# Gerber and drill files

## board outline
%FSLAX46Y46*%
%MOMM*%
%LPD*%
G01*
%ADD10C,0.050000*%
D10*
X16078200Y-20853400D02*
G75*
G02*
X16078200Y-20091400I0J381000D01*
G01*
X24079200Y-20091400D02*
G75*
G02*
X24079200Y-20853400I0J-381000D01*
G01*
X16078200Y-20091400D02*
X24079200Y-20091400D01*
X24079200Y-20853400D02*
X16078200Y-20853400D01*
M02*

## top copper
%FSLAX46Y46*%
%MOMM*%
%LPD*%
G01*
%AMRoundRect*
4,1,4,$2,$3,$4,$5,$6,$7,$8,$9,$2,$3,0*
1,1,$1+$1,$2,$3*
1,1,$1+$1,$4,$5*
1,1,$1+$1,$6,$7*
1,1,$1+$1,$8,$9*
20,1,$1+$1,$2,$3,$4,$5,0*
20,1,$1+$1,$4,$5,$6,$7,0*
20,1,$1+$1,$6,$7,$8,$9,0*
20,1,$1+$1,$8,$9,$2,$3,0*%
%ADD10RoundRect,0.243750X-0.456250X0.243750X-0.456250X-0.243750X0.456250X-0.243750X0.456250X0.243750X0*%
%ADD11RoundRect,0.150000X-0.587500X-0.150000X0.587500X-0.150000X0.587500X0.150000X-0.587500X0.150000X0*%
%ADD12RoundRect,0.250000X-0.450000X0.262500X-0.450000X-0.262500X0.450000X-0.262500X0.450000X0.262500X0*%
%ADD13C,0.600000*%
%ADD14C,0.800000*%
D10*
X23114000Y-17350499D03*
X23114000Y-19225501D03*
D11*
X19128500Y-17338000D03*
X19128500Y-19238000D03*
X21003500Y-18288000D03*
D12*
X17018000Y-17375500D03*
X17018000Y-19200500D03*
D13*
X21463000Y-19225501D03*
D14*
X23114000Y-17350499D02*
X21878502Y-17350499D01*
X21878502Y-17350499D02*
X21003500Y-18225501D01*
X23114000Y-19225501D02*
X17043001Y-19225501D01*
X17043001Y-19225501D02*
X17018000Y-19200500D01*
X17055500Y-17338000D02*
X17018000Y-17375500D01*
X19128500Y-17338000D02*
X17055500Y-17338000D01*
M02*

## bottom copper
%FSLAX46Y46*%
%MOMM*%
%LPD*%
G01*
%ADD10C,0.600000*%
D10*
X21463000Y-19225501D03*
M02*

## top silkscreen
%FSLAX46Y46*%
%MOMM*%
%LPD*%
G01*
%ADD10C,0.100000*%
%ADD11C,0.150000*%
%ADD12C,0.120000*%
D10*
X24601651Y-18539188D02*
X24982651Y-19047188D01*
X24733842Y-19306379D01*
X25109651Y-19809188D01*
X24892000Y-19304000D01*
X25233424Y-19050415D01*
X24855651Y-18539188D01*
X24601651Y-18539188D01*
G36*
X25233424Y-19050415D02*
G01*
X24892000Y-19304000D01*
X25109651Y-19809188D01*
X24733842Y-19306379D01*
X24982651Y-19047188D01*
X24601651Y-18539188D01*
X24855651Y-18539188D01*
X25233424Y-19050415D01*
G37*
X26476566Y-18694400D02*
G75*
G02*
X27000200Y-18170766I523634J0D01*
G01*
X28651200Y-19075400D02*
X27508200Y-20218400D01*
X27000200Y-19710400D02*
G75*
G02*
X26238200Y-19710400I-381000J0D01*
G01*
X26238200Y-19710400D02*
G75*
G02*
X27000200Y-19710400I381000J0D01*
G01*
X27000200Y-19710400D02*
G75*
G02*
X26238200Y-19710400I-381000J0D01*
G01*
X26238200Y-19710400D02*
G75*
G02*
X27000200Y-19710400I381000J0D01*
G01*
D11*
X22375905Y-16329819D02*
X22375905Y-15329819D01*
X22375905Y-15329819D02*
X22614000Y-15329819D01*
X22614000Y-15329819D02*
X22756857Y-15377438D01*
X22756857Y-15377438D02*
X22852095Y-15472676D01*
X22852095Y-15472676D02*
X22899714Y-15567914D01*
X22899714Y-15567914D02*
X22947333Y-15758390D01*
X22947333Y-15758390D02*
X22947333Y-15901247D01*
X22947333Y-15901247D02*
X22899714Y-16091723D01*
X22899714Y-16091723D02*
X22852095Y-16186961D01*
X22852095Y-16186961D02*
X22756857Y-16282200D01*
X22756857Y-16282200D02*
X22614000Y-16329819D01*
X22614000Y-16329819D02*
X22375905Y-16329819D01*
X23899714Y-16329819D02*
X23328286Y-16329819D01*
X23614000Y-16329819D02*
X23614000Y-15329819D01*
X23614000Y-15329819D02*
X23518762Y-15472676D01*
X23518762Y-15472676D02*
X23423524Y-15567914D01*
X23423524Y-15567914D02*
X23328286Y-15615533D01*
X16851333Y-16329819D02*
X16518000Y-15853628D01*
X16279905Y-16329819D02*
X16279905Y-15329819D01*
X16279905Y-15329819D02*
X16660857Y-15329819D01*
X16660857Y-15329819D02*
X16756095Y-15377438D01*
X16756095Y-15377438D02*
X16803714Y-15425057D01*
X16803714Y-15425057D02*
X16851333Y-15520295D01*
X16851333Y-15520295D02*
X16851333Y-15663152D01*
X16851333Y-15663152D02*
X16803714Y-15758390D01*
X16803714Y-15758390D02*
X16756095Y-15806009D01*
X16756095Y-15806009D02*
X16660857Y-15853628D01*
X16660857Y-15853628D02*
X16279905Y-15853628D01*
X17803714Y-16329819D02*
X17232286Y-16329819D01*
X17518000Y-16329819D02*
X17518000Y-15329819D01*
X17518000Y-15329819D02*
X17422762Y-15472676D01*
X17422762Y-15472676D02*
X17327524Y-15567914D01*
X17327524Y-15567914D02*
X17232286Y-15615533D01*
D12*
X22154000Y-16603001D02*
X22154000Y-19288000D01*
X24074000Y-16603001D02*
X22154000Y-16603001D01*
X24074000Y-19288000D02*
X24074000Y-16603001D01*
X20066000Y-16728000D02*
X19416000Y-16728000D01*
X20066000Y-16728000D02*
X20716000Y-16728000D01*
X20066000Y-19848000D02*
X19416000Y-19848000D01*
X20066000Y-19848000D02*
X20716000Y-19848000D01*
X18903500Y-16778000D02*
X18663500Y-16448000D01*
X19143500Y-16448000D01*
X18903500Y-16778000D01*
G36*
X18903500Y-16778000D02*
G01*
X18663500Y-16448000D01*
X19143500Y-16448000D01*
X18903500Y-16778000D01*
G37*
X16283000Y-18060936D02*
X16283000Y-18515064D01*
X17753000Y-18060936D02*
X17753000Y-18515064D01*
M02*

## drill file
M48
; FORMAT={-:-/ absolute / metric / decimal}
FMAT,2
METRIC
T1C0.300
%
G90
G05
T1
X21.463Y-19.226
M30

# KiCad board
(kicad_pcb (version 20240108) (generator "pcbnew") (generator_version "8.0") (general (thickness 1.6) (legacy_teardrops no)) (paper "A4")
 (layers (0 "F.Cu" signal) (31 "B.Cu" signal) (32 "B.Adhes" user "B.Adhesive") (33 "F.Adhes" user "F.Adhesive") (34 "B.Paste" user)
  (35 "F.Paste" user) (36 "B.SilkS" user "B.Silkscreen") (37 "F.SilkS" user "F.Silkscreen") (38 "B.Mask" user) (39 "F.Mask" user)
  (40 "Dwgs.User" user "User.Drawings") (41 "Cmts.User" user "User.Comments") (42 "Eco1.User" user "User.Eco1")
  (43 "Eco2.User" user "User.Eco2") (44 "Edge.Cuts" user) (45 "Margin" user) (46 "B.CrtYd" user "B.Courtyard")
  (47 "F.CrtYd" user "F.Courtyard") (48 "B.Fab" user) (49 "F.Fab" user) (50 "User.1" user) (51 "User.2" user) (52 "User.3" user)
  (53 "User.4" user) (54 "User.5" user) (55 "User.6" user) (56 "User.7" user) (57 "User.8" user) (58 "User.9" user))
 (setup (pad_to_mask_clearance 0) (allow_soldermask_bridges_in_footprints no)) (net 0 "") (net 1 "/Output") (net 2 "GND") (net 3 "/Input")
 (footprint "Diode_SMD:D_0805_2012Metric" (layer "F.Cu") (at 23.114 18.288 -90)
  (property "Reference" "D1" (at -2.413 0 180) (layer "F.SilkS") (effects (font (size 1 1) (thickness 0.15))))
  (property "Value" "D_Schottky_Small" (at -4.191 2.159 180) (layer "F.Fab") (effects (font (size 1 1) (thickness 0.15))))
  (fp_line (start -1.684999 0.96) (end 1 0.96) (stroke (width 0.12) (type solid)) (layer "F.SilkS"))
  (fp_line (start -1.684999 -0.96) (end -1.684999 0.96) (stroke (width 0.12) (type solid)) (layer "F.SilkS"))
  (fp_line (start 1 -0.96) (end -1.684999 -0.96) (stroke (width 0.12) (type solid)) (layer "F.SilkS"))
  (pad "1" smd roundrect (at -0.937501 0 270) (size 0.975 1.4) (layers "F.Cu" "F.Paste" "F.Mask") (roundrect_rratio 0.25) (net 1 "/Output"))
  (pad "2" smd roundrect (at 0.937501 0 270) (size 0.975 1.4) (layers "F.Cu" "F.Paste" "F.Mask") (roundrect_rratio 0.25) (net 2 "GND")))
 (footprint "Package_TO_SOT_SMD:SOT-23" (layer "F.Cu") (at 20.066 18.288)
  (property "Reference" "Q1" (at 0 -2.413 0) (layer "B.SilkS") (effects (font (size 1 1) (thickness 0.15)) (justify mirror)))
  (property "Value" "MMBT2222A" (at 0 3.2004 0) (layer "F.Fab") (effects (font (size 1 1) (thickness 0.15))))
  (fp_line (start 0 -1.56) (end -0.65 -1.56) (stroke (width 0.12) (type solid)) (layer "F.SilkS"))
  (fp_line (start 0 -1.56) (end 0.65 -1.56) (stroke (width 0.12) (type solid)) (layer "F.SilkS"))
  (fp_line (start 0 1.56) (end -0.65 1.56) (stroke (width 0.12) (type solid)) (layer "F.SilkS"))
  (fp_line (start 0 1.56) (end 0.65 1.56) (stroke (width 0.12) (type solid)) (layer "F.SilkS"))
  (fp_poly
   (pts (xy -1.1625 -1.51) (xy -1.4025 -1.84) (xy -0.9225 -1.84) (xy -1.1625 -1.51)) (stroke (width 0.12) (type solid)) (fill solid)
   (layer "F.SilkS"))
  (pad "1" smd roundrect (at -0.9375 -0.95) (size 1.475 0.6) (layers "F.Cu" "F.Paste" "F.Mask") (roundrect_rratio 0.25) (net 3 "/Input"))
  (pad "2" smd roundrect (at -0.9375 0.95) (size 1.475 0.6) (layers "F.Cu" "F.Paste" "F.Mask") (roundrect_rratio 0.25) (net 2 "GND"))
  (pad "3" smd roundrect (at 0.9375 0) (size 1.475 0.6) (layers "F.Cu" "F.Paste" "F.Mask") (roundrect_rratio 0.25) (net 1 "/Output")))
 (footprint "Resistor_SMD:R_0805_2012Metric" (layer "F.Cu") (at 17.018 18.288 -90)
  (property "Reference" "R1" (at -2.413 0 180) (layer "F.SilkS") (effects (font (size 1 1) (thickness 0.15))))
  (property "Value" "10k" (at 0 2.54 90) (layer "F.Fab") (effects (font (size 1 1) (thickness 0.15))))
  (fp_line (start -0.227064 0.735) (end 0.227064 0.735) (stroke (width 0.12) (type solid)) (layer "F.SilkS"))
  (fp_line (start -0.227064 -0.735) (end 0.227064 -0.735) (stroke (width 0.12) (type solid)) (layer "F.SilkS"))
  (pad "1" smd roundrect (at -0.9125 0 270) (size 1.025 1.4) (layers "F.Cu" "F.Paste" "F.Mask") (roundrect_rratio 0.243902) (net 3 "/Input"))
  (pad "2" smd roundrect (at 0.9125 0 270) (size 1.025 1.4) (layers "F.Cu" "F.Paste" "F.Mask") (roundrect_rratio 0.243902) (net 2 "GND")))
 (gr_poly
  (pts (xy 24.601651 18.539188) (xy 24.982651 19.047188) (xy 24.733842 19.306379) (xy 25.109651 19.809188) (xy 24.892 19.304)
   (xy 25.233424 19.050415) (xy 24.855651 18.539188))
  (stroke (width 0.1) (type solid)) (fill solid) (layer "F.SilkS"))
 (gr_arc (start 26.476566 18.6944) (mid 26.629935 18.324135) (end 27.0002 18.170766) (stroke (width 0.1) (type default)) (layer "F.SilkS"))
 (gr_line (start 28.6512 19.0754) (end 27.5082 20.2184) (stroke (width 0.1) (type default)) (layer "F.SilkS"))
 (gr_circle (center 26.6192 19.7104) (end 26.6192 19.3294) (stroke (width 0.1) (type default)) (fill none) (layer "F.SilkS"))
 (gr_circle (center 26.6192 19.7104) (end 26.6192 19.3294) (stroke (width 0.1) (type default)) (fill none) (layer "F.SilkS"))
 (gr_arc (start 16.0782 20.8534) (mid 15.6972 20.4724) (end 16.0782 20.0914) (stroke (width 0.05) (type default)) (layer "Edge.Cuts"))
 (gr_arc (start 24.0792 20.0914) (mid 24.4602 20.4724) (end 24.0792 20.8534) (stroke (width 0.05) (type default)) (layer "Edge.Cuts"))
 (gr_line (start 16.0782 20.0914) (end 24.0792 20.0914) (stroke (width 0.05) (type default)) (layer "Edge.Cuts"))
 (gr_line (start 24.0792 20.8534) (end 16.0782 20.8534) (stroke (width 0.05) (type default)) (layer "Edge.Cuts"))
 (segment (start 23.114 17.350499) (end 21.878502 17.350499) (width 0.8) (layer "F.Cu") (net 1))
 (segment (start 21.878502 17.350499) (end 21.0035 18.225501) (width 0.8) (layer "F.Cu") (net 1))
 (segment (start 23.114 19.225501) (end 17.043001 19.225501) (width 0.8) (layer "F.Cu") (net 2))
 (segment (start 17.043001 19.225501) (end 17.018 19.2005) (width 0.8) (layer "F.Cu") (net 2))
 (via (at 21.463 19.225501) (size 0.6) (drill 0.3) (layers "F.Cu" "B.Cu") (free yes) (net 2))
 (segment (start 17.0555 17.338) (end 17.018 17.3755) (width 0.8) (layer "F.Cu") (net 3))
 (segment (start 19.1285 17.338) (end 17.0555 17.338) (width 0.8) (layer "F.Cu") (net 3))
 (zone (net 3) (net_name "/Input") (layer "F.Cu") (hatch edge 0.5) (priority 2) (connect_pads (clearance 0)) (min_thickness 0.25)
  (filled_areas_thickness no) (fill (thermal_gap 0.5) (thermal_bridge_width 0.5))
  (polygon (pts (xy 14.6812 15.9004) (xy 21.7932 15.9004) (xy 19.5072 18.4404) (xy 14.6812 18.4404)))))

